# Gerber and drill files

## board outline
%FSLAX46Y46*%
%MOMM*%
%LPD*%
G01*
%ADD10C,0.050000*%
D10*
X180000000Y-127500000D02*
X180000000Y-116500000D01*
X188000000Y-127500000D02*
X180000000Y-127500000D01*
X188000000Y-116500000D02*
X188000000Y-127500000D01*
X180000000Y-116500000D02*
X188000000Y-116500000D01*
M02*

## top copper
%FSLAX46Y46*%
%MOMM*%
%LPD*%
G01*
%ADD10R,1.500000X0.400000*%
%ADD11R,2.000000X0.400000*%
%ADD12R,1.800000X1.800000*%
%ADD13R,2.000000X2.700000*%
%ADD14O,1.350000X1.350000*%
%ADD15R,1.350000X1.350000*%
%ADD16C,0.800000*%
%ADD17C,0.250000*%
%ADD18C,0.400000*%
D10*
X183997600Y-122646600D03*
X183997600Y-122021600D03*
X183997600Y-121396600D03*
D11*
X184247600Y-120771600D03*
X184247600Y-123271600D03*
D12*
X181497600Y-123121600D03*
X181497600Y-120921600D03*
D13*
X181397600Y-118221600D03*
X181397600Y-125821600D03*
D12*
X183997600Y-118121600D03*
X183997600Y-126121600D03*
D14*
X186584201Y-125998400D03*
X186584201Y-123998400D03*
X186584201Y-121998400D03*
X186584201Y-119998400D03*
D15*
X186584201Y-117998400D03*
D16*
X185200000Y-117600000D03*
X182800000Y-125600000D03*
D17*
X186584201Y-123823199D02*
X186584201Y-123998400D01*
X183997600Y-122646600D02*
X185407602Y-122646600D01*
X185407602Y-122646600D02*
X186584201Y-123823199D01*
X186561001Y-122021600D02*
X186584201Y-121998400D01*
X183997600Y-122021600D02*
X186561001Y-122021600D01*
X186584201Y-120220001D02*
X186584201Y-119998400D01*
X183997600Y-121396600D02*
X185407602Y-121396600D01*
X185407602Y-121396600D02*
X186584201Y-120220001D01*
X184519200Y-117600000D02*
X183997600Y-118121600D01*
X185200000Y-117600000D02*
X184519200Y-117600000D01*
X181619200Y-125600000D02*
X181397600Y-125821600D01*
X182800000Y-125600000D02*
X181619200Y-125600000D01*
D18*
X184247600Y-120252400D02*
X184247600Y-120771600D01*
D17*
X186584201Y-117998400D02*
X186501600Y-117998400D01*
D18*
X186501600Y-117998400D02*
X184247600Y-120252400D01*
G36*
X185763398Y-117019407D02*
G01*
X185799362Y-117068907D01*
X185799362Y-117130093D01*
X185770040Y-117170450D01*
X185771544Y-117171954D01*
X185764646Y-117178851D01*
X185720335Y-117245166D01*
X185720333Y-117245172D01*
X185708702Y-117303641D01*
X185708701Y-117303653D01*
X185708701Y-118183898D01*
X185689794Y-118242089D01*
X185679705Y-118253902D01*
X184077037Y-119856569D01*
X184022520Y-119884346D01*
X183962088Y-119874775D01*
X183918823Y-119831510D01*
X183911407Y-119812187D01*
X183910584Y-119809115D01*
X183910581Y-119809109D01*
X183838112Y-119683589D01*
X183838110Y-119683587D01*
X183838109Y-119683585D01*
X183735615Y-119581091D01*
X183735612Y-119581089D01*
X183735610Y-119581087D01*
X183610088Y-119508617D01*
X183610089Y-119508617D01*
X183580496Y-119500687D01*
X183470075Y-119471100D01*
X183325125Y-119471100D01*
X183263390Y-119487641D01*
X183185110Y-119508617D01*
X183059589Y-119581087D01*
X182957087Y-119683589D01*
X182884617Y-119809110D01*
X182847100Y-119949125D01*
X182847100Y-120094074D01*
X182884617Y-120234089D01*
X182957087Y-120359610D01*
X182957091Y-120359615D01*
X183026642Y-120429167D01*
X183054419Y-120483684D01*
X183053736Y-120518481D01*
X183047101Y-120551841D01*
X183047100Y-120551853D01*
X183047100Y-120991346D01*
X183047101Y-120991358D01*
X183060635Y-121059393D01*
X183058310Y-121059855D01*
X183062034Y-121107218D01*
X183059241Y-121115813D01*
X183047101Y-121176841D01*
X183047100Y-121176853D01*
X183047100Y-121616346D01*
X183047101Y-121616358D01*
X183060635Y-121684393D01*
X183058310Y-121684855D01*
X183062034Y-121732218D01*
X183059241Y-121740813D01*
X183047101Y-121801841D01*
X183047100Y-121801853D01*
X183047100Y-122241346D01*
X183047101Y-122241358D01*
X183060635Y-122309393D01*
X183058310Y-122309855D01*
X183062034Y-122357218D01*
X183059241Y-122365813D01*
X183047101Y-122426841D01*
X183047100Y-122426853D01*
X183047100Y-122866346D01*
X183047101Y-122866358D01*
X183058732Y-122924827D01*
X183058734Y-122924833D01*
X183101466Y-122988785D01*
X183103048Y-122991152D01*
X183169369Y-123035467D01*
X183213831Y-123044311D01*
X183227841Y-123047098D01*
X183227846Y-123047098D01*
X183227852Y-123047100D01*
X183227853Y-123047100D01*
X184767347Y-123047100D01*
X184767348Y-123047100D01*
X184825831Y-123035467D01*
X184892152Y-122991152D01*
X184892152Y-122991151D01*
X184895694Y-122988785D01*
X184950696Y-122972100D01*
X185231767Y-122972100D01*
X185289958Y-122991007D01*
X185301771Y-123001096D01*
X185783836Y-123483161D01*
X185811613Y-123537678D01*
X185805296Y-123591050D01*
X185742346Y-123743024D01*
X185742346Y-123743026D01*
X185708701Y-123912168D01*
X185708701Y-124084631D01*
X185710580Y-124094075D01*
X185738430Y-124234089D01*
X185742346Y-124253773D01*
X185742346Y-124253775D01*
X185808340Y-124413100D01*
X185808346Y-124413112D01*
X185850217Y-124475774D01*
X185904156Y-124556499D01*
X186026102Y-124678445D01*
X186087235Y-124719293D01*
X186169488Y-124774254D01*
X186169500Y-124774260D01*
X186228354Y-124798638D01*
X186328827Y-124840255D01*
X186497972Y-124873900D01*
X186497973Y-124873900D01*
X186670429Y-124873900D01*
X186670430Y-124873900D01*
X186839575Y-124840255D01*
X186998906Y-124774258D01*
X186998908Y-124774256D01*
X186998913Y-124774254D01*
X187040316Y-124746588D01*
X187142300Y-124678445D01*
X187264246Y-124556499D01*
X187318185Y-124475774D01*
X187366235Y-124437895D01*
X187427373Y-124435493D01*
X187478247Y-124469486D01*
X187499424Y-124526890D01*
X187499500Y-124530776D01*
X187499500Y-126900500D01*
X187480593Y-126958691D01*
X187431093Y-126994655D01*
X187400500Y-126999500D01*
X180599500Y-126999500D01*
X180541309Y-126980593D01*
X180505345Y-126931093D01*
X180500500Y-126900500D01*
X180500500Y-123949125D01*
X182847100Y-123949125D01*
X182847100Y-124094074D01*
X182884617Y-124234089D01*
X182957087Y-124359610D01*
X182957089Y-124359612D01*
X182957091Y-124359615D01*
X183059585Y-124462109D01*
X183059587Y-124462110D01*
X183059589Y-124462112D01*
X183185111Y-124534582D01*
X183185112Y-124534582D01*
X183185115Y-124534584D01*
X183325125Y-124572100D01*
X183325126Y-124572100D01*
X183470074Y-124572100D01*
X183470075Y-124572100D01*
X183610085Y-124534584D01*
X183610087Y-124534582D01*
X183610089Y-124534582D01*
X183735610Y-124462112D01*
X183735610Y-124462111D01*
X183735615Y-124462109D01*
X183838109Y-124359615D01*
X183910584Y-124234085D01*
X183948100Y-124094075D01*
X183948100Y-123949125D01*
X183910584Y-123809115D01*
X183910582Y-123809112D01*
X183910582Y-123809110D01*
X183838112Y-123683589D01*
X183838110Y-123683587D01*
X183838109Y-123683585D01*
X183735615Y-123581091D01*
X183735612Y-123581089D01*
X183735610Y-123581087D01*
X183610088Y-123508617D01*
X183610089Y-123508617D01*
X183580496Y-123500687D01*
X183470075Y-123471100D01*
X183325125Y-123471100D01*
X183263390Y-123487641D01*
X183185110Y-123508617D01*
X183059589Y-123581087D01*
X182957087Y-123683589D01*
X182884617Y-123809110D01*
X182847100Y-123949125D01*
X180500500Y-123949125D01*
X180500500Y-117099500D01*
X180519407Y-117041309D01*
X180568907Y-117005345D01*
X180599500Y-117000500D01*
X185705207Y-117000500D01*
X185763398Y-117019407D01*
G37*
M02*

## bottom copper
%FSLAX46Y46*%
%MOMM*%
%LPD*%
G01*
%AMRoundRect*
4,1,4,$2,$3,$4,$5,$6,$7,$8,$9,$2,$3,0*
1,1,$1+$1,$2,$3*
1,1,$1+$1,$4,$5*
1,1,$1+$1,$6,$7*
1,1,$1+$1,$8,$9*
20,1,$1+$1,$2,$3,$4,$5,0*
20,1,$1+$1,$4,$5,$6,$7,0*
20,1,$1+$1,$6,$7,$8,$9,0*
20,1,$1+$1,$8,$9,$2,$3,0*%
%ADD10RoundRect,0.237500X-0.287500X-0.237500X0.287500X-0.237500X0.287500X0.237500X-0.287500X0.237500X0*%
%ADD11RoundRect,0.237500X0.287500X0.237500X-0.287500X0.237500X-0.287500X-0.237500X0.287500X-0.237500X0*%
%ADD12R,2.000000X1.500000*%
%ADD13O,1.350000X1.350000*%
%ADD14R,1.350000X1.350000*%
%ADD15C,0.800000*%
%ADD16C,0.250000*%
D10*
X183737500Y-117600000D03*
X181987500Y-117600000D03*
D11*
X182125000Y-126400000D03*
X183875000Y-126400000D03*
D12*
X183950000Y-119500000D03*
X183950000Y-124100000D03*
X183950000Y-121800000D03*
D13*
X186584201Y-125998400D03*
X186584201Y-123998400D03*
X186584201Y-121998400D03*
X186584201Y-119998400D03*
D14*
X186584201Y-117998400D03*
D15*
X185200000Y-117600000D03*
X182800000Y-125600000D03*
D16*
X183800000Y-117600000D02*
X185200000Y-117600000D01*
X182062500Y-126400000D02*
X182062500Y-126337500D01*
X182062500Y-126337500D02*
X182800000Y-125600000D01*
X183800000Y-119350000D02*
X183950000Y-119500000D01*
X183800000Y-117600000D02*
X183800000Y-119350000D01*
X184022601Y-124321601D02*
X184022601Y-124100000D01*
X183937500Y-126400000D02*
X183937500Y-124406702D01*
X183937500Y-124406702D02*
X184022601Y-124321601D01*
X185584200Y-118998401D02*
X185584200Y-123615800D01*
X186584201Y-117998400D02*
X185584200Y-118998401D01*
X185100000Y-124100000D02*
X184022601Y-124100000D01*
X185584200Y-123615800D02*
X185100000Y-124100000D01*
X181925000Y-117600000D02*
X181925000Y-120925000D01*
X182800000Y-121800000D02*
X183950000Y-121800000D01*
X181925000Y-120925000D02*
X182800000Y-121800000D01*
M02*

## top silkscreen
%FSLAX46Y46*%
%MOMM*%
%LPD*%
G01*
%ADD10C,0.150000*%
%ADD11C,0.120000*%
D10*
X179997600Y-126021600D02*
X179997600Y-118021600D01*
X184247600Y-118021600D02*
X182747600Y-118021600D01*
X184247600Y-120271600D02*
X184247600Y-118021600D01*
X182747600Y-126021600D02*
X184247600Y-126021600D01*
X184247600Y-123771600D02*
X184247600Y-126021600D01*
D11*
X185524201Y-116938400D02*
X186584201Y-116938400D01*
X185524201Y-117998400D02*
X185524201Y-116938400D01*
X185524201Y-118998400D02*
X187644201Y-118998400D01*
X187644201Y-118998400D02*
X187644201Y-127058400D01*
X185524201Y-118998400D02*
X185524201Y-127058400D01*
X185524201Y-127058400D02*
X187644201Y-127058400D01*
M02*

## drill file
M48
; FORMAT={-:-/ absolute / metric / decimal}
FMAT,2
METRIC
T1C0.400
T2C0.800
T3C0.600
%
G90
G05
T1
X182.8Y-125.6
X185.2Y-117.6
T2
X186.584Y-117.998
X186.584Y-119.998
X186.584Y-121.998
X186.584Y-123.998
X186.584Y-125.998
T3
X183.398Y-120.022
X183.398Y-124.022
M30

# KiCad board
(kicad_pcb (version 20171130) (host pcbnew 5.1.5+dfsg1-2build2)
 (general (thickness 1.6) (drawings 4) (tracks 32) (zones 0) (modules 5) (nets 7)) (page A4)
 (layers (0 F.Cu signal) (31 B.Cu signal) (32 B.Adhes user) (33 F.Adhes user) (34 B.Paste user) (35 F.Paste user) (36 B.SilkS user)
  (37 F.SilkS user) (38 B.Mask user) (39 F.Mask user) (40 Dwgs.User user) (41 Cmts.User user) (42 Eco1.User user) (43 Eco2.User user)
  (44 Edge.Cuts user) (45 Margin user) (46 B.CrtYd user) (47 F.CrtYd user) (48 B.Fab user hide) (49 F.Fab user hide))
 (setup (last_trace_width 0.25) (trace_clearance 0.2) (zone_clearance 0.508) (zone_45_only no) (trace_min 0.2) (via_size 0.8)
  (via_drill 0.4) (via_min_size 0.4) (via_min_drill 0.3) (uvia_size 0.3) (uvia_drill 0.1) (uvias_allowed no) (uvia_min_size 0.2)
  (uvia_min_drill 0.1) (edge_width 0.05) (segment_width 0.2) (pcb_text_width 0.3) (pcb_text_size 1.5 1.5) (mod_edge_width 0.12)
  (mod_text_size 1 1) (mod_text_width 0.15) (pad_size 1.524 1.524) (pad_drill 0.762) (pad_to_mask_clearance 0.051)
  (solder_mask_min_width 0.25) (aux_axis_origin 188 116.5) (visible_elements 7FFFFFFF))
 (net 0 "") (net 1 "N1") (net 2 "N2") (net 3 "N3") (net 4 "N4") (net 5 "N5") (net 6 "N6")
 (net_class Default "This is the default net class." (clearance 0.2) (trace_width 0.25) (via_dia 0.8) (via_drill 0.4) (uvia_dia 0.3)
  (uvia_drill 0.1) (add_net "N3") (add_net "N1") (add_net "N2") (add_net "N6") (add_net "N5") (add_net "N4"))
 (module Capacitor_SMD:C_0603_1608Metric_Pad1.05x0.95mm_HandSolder (layer B.Cu) (at 182.8625 117.6)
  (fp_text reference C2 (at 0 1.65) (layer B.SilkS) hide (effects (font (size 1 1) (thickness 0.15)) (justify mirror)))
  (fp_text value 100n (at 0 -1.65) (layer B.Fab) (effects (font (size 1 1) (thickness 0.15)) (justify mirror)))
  (pad 2 smd roundrect (at 0.875 0) (size 1.05 0.95) (layers B.Cu B.Paste B.Mask) (roundrect_rratio 0.25) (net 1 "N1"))
  (pad 1 smd roundrect (at -0.875 0) (size 1.05 0.95) (layers B.Cu B.Paste B.Mask) (roundrect_rratio 0.25) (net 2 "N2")))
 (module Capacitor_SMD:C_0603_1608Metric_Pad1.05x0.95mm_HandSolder (layer B.Cu) (at 183 126.4 180)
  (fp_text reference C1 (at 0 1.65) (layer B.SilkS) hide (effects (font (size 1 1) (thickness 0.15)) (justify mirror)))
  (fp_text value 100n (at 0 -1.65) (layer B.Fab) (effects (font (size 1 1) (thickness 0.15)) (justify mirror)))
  (pad 2 smd roundrect (at 0.875 0 180) (size 1.05 0.95) (layers B.Cu B.Paste B.Mask) (roundrect_rratio 0.25) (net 1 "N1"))
  (pad 1 smd roundrect (at -0.875 0 180) (size 1.05 0.95) (layers B.Cu B.Paste B.Mask) (roundrect_rratio 0.25) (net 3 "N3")))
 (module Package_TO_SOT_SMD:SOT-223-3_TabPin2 (layer B.Cu) (at 180.8 121.8 180)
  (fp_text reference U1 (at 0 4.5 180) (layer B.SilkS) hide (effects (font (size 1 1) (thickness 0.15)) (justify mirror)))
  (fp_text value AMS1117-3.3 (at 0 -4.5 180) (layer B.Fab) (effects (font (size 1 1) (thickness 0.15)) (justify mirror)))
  (pad 1 smd rect (at -3.15 2.3 180) (size 2 1.5) (layers B.Cu B.Paste B.Mask) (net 1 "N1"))
  (pad 3 smd rect (at -3.15 -2.3 180) (size 2 1.5) (layers B.Cu B.Paste B.Mask) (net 3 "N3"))
  (pad 2 smd rect (at -3.15 0 180) (size 2 1.5) (layers B.Cu B.Paste B.Mask) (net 2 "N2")))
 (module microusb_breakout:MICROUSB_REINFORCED (layer F.Cu) (at 183.9976 122.0216 90) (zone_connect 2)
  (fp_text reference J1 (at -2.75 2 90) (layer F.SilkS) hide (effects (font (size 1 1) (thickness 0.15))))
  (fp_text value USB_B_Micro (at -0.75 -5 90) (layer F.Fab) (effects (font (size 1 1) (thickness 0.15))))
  (fp_line (start -4 -4) (end 4 -4) (layer F.SilkS) (width 0.15))
  (fp_line (start 4 0.25) (end 4 -1.25) (layer F.SilkS) (width 0.15))
  (fp_line (start 1.75 0.25) (end 4 0.25) (layer F.SilkS) (width 0.15))
  (fp_line (start -4 -1.25) (end -4 0.25) (layer F.SilkS) (width 0.15))
  (fp_line (start -1.75 0.25) (end -4 0.25) (layer F.SilkS) (width 0.15))
  (pad 4 smd rect (at -0.625 0 90) (size 0.4 1.5) (layers F.Cu F.Paste F.Mask) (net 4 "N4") (zone_connect 2))
  (pad 3 smd rect (at 0 0 90) (size 0.4 1.5) (layers F.Cu F.Paste F.Mask) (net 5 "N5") (zone_connect 2))
  (pad 2 smd rect (at 0.625 0 90) (size 0.4 1.5) (layers F.Cu F.Paste F.Mask) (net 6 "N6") (zone_connect 2))
  (pad 1 smd rect (at 1.25 0.25 90) (size 0.4 2) (layers F.Cu F.Paste F.Mask) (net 3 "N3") (zone_connect 2))
  (pad 5 smd rect (at -1.25 0.25 90) (size 0.4 2) (layers F.Cu F.Paste F.Mask) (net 1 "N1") (zone_connect 2))
  (pad 6 smd rect (at -1.1 -2.5 90) (size 1.8 1.8) (layers F.Cu F.Paste F.Mask) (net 1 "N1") (zone_connect 2))
  (pad 6 smd rect (at 1.1 -2.5 90) (size 1.8 1.8) (layers F.Cu F.Paste F.Mask) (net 1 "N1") (zone_connect 2))
  (pad 6 smd rect (at 3.8 -2.6 90) (size 2.7 2) (layers F.Cu F.Paste F.Mask) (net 1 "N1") (zone_connect 2))
  (pad 6 smd rect (at -3.8 -2.6 90) (size 2.7 2) (layers F.Cu F.Paste F.Mask) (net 1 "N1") (zone_connect 2))
  (pad "" np_thru_hole circle (at 2 -0.6 90) (size 0.6 0.6) (drill 0.6) (layers *.Cu *.Mask) (zone_connect 2))
  (pad "" np_thru_hole circle (at -2 -0.6 90) (size 0.6 0.6) (drill 0.6) (layers *.Cu *.Mask) (zone_connect 2))
  (pad 6 smd rect (at 3.9 0 90) (size 1.8 1.8) (layers F.Cu F.Paste F.Mask) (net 1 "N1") (zone_connect 2))
  (pad 6 smd rect (at -4.1 0 90) (size 1.8 1.8) (layers F.Cu F.Paste F.Mask) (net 1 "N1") (zone_connect 2)))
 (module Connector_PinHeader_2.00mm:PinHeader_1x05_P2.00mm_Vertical (layer F.Cu) (at 186.584201 117.9984)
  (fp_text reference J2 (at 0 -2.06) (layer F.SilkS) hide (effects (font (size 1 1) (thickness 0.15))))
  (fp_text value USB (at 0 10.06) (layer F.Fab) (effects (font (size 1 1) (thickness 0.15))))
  (fp_line (start -1.06 -1.06) (end 0 -1.06) (layer F.SilkS) (width 0.12))
  (fp_line (start -1.06 0) (end -1.06 -1.06) (layer F.SilkS) (width 0.12))
  (fp_line (start -1.06 1) (end 1.06 1) (layer F.SilkS) (width 0.12))
  (fp_line (start 1.06 1) (end 1.06 9.06) (layer F.SilkS) (width 0.12))
  (fp_line (start -1.06 1) (end -1.06 9.06) (layer F.SilkS) (width 0.12))
  (fp_line (start -1.06 9.06) (end 1.06 9.06) (layer F.SilkS) (width 0.12))
  (pad 5 thru_hole oval (at 0 8) (size 1.35 1.35) (drill 0.8) (layers *.Cu *.Mask) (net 1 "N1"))
  (pad 4 thru_hole oval (at 0 6) (size 1.35 1.35) (drill 0.8) (layers *.Cu *.Mask) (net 4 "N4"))
  (pad 3 thru_hole oval (at 0 4) (size 1.35 1.35) (drill 0.8) (layers *.Cu *.Mask) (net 5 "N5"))
  (pad 2 thru_hole oval (at 0 2) (size 1.35 1.35) (drill 0.8) (layers *.Cu *.Mask) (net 6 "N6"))
  (pad 1 thru_hole rect (at 0 0) (size 1.35 1.35) (drill 0.8) (layers *.Cu *.Mask) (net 3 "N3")))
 (gr_line (start 180 127.5) (end 180 116.5) (layer Edge.Cuts) (width 0.05))
 (gr_line (start 188 127.5) (end 180 127.5) (layer Edge.Cuts) (width 0.05))
 (gr_line (start 188 116.5) (end 188 127.5) (layer Edge.Cuts) (width 0.05))
 (gr_line (start 180 116.5) (end 188 116.5) (layer Edge.Cuts) (width 0.05))
 (segment (start 186.584201 123.823199) (end 186.584201 123.9984) (width 0.25) (layer F.Cu) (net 4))
 (segment (start 183.9976 122.6466) (end 185.407602 122.6466) (width 0.25) (layer F.Cu) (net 4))
 (segment (start 185.407602 122.6466) (end 186.584201 123.823199) (width 0.25) (layer F.Cu) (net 4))
 (segment (start 186.561001 122.0216) (end 186.584201 121.9984) (width 0.25) (layer F.Cu) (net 5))
 (segment (start 183.9976 122.0216) (end 186.561001 122.0216) (width 0.25) (layer F.Cu) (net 5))
 (segment (start 186.584201 120.220001) (end 186.584201 119.9984) (width 0.25) (layer F.Cu) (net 6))
 (segment (start 183.9976 121.3966) (end 185.407602 121.3966) (width 0.25) (layer F.Cu) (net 6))
 (segment (start 185.407602 121.3966) (end 186.584201 120.220001) (width 0.25) (layer F.Cu) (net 6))
 (via (at 185.2 117.6) (size 0.8) (drill 0.4) (layers F.Cu B.Cu) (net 1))
 (segment (start 183.8 117.6) (end 185.2 117.6) (width 0.25) (layer B.Cu) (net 1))
 (segment (start 184.5192 117.6) (end 183.9976 118.1216) (width 0.25) (layer F.Cu) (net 1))
 (segment (start 185.2 117.6) (end 184.5192 117.6) (width 0.25) (layer F.Cu) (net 1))
 (via (at 182.8 125.6) (size 0.8) (drill 0.4) (layers F.Cu B.Cu) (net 1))
 (segment (start 182.0625 126.4) (end 182.0625 126.3375) (width 0.25) (layer B.Cu) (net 1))
 (segment (start 182.0625 126.3375) (end 182.8 125.6) (width 0.25) (layer B.Cu) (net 1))
 (segment (start 181.6192 125.6) (end 181.3976 125.8216) (width 0.25) (layer F.Cu) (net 1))
 (segment (start 182.8 125.6) (end 181.6192 125.6) (width 0.25) (layer F.Cu) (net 1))
 (segment (start 183.8 119.35) (end 183.95 119.5) (width 0.25) (layer B.Cu) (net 1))
 (segment (start 183.8 117.6) (end 183.8 119.35) (width 0.25) (layer B.Cu) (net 1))
 (segment (start 184.2476 120.2524) (end 184.2476 120.7716) (width 0.4) (layer F.Cu) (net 3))
 (segment (start 186.584201 117.9984) (end 186.5016 117.9984) (width 0.25) (layer F.Cu) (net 3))
 (segment (start 186.5016 117.9984) (end 184.2476 120.2524) (width 0.4) (layer F.Cu) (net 3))
 (segment (start 184.022601 124.321601) (end 184.022601 124.1) (width 0.25) (layer B.Cu) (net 3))
 (segment (start 183.9375 126.4) (end 183.9375 124.406702) (width 0.25) (layer B.Cu) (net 3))
 (segment (start 183.9375 124.406702) (end 184.022601 124.321601) (width 0.25) (layer B.Cu) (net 3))
 (segment (start 185.5842 118.998401) (end 185.5842 123.6158) (width 0.25) (layer B.Cu) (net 3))
 (segment (start 186.584201 117.9984) (end 185.5842 118.998401) (width 0.25) (layer B.Cu) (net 3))
 (segment (start 185.1 124.1) (end 184.022601 124.1) (width 0.25) (layer B.Cu) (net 3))
 (segment (start 185.5842 123.6158) (end 185.1 124.1) (width 0.25) (layer B.Cu) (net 3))
 (segment (start 181.925 117.6) (end 181.925 120.925) (width 0.25) (layer B.Cu) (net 2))
 (segment (start 182.8 121.8) (end 183.95 121.8) (width 0.25) (layer B.Cu) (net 2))
 (segment (start 181.925 120.925) (end 182.8 121.8) (width 0.25) (layer B.Cu) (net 2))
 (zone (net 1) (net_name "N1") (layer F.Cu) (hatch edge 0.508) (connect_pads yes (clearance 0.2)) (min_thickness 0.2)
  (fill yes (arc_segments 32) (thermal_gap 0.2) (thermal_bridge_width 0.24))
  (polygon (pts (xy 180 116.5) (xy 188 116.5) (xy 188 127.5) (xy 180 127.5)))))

